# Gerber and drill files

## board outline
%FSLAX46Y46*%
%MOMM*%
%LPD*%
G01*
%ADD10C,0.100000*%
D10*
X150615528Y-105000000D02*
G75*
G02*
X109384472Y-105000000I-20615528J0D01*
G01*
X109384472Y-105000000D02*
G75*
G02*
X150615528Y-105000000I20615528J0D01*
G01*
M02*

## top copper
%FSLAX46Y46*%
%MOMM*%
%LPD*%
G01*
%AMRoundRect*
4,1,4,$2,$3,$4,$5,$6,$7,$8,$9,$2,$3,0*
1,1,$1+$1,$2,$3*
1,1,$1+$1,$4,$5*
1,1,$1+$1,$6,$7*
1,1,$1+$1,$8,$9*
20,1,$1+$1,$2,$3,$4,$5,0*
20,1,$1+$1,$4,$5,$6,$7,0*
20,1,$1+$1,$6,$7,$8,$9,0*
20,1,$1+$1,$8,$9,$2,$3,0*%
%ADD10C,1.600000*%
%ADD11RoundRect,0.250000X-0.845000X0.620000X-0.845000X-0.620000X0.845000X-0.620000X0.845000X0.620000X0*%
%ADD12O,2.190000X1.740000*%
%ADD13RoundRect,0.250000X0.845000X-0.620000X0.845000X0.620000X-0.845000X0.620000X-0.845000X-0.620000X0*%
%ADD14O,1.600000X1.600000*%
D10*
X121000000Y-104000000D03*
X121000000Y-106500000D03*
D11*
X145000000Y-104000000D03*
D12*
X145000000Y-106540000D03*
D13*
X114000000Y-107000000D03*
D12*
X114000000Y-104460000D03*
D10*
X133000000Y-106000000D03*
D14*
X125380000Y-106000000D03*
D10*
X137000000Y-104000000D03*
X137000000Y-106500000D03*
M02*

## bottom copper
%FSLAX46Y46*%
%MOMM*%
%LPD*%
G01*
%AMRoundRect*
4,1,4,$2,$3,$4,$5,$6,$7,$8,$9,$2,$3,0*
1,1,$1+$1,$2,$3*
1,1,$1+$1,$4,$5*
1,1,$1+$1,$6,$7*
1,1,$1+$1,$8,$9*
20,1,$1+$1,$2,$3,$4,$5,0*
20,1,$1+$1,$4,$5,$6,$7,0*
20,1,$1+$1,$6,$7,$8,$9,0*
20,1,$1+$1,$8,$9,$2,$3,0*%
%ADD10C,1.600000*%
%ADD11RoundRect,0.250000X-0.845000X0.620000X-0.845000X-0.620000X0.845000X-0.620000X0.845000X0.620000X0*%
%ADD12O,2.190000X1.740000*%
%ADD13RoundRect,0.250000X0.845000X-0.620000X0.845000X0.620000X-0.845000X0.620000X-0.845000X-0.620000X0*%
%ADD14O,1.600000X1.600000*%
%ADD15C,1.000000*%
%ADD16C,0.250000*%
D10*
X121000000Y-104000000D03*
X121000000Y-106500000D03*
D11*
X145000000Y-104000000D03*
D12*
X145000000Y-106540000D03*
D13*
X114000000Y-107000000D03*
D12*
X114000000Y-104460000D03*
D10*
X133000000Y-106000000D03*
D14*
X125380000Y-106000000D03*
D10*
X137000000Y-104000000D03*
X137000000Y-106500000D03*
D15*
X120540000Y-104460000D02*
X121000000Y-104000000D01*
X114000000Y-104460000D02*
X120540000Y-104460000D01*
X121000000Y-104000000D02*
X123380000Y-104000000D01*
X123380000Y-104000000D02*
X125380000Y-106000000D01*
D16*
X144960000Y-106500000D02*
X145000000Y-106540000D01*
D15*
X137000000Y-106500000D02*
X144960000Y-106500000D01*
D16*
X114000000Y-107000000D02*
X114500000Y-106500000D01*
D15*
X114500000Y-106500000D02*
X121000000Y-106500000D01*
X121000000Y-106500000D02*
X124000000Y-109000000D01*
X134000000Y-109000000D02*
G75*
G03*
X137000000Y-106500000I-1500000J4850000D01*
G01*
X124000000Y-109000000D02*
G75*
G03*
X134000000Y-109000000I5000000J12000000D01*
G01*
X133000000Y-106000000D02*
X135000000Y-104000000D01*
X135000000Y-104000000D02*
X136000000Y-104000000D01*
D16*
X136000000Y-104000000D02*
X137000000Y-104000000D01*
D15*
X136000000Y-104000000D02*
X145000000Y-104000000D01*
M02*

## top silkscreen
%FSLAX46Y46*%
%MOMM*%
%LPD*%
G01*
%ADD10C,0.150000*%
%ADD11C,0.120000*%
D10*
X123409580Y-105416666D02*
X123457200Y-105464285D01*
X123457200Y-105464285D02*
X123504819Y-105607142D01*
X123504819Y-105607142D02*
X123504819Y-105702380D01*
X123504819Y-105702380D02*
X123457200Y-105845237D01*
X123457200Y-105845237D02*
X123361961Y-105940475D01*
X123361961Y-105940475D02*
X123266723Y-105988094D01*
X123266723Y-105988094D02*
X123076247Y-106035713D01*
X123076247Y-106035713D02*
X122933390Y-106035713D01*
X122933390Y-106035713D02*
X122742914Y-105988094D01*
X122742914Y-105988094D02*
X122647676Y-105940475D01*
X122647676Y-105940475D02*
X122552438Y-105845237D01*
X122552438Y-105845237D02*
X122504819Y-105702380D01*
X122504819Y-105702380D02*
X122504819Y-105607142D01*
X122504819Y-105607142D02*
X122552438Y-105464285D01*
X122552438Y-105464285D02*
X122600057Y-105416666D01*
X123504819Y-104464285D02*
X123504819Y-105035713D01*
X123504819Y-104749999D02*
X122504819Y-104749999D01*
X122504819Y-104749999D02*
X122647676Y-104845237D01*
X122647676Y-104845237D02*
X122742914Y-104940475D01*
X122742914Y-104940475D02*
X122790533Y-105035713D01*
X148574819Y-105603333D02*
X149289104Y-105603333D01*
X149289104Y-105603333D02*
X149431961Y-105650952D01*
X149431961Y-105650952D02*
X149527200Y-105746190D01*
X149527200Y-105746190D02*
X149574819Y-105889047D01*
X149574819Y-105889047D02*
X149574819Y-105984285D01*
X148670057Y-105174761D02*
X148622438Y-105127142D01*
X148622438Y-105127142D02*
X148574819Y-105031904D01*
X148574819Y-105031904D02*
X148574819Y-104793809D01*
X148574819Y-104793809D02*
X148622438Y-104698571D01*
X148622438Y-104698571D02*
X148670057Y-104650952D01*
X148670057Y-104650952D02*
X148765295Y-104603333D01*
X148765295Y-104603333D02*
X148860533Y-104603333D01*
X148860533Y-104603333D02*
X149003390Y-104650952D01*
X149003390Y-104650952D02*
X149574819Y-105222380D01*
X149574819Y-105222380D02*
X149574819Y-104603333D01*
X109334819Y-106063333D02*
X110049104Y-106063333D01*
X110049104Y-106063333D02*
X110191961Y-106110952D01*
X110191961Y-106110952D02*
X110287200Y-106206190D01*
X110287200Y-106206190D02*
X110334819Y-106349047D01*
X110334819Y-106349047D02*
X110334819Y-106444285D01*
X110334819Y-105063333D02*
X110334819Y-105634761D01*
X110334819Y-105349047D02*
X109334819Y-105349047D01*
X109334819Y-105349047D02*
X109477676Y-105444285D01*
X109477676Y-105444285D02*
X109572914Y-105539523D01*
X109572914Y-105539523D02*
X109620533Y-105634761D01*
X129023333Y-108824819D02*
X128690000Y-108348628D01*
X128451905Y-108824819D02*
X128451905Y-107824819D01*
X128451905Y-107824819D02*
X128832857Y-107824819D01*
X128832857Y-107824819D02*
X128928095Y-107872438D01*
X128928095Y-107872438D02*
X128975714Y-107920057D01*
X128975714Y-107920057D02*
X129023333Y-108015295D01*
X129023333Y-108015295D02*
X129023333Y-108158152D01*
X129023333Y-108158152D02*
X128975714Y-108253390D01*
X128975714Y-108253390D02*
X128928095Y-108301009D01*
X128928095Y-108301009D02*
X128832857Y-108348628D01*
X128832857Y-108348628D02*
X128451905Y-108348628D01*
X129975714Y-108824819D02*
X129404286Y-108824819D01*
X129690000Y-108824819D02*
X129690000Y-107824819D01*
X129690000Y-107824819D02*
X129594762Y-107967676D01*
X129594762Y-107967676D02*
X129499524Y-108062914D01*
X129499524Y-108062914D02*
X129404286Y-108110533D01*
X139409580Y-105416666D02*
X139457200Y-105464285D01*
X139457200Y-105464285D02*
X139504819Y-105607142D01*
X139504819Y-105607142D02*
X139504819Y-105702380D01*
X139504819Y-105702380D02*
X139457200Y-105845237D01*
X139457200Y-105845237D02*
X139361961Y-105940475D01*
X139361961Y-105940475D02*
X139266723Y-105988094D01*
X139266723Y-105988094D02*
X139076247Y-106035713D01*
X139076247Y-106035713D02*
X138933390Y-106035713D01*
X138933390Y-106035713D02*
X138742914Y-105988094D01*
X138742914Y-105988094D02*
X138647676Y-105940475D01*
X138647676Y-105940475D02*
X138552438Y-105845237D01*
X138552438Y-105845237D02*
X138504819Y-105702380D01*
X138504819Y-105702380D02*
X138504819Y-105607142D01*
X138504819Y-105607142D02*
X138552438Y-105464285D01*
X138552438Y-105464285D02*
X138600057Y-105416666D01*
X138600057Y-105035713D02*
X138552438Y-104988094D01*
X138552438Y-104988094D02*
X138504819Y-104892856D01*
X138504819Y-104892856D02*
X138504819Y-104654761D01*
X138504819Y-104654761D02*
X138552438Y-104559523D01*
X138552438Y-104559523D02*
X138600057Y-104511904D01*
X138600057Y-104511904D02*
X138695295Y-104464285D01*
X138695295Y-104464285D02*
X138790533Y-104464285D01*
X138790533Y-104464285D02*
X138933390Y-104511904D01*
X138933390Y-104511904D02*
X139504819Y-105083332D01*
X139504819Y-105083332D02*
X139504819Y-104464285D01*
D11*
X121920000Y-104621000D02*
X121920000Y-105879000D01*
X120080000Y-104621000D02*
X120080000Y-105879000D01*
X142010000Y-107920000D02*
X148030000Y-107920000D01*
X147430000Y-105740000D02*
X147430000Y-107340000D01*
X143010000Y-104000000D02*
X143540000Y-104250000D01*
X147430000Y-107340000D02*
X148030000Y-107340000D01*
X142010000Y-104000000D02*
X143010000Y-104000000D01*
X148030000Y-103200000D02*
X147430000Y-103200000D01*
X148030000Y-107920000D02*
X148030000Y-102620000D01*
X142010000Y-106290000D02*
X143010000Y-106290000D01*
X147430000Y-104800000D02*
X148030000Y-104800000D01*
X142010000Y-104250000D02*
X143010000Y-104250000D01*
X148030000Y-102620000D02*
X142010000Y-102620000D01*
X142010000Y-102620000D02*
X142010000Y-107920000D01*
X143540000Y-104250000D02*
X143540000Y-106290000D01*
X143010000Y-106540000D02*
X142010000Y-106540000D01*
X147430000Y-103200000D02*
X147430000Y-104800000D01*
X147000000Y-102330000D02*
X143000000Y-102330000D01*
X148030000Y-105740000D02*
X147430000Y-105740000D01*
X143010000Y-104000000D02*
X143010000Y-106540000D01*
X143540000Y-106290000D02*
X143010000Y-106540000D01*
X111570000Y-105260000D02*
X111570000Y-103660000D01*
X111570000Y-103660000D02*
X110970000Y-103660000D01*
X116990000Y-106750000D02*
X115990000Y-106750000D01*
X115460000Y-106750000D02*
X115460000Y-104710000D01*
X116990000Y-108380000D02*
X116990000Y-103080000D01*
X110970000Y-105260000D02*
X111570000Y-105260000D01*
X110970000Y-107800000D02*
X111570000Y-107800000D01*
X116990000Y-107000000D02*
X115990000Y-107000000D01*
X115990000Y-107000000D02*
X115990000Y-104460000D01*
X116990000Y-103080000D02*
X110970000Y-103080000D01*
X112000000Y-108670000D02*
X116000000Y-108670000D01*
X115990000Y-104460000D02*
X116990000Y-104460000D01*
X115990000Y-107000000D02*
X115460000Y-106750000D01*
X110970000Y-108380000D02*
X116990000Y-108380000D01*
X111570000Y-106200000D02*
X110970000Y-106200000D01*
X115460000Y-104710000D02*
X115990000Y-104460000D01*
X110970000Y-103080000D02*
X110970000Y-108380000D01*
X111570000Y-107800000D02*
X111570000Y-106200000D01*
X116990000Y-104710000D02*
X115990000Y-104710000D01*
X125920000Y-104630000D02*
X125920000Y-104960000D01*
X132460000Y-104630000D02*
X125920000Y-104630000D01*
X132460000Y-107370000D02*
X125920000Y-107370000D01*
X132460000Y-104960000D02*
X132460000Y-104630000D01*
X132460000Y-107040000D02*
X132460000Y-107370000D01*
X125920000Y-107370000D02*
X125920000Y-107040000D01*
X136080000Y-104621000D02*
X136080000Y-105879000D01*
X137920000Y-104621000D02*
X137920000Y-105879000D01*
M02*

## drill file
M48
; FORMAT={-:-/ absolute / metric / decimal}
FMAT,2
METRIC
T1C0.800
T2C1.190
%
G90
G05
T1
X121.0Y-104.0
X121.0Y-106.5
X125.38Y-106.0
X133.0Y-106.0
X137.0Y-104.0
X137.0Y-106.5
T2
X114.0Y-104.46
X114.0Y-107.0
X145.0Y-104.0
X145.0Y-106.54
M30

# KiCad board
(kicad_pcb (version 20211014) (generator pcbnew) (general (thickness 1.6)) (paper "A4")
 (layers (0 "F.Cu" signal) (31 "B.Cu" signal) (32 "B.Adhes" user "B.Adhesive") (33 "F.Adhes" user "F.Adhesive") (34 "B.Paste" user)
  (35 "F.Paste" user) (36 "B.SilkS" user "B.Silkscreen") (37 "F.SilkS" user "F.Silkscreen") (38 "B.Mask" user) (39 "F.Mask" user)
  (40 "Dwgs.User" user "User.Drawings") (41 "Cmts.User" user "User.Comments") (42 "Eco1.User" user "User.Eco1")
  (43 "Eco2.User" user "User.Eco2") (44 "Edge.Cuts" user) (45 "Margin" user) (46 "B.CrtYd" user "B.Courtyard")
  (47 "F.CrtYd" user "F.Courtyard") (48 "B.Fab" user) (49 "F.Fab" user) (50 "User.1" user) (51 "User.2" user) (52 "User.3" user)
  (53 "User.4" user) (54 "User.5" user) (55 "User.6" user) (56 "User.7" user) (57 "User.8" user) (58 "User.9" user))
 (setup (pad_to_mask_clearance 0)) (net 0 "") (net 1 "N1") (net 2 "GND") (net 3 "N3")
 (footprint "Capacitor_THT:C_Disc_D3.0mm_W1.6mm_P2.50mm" (layer "F.Cu") (at 121 104 -90)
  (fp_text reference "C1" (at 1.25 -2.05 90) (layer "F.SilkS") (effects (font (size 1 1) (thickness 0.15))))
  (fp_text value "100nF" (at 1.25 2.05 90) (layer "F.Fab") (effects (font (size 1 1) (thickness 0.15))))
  (fp_line (start 0.621 -0.92) (end 1.879 -0.92) (layer "F.SilkS") (width 0.12))
  (fp_line (start 0.621 0.92) (end 1.879 0.92) (layer "F.SilkS") (width 0.12))
  (pad "1" thru_hole circle (at 0 0 270) (size 1.6 1.6) (drill 0.8) (layers *.Cu *.Mask) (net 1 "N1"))
  (pad "2" thru_hole circle (at 2.5 0 270) (size 1.6 1.6) (drill 0.8) (layers *.Cu *.Mask) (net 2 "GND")))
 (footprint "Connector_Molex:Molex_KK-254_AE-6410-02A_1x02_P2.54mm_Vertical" (layer "F.Cu") (at 145 104 -90)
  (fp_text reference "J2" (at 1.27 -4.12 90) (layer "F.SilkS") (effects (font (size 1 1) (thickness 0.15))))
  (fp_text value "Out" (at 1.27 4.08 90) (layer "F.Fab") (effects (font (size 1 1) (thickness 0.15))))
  (fp_line (start 3.92 2.99) (end 3.92 -3.03) (layer "F.SilkS") (width 0.12))
  (fp_line (start 1.74 -2.43) (end 3.34 -2.43) (layer "F.SilkS") (width 0.12))
  (fp_line (start 0 1.99) (end 0.25 1.46) (layer "F.SilkS") (width 0.12))
  (fp_line (start 3.34 -2.43) (end 3.34 -3.03) (layer "F.SilkS") (width 0.12))
  (fp_line (start 0 2.99) (end 0 1.99) (layer "F.SilkS") (width 0.12))
  (fp_line (start -0.8 -3.03) (end -0.8 -2.43) (layer "F.SilkS") (width 0.12))
  (fp_line (start 3.92 -3.03) (end -1.38 -3.03) (layer "F.SilkS") (width 0.12))
  (fp_line (start 2.29 2.99) (end 2.29 1.99) (layer "F.SilkS") (width 0.12))
  (fp_line (start 0.8 -2.43) (end 0.8 -3.03) (layer "F.SilkS") (width 0.12))
  (fp_line (start 0.25 2.99) (end 0.25 1.99) (layer "F.SilkS") (width 0.12))
  (fp_line (start -1.38 -3.03) (end -1.38 2.99) (layer "F.SilkS") (width 0.12))
  (fp_line (start -1.38 2.99) (end 3.92 2.99) (layer "F.SilkS") (width 0.12))
  (fp_line (start 0.25 1.46) (end 2.29 1.46) (layer "F.SilkS") (width 0.12))
  (fp_line (start 2.54 1.99) (end 2.54 2.99) (layer "F.SilkS") (width 0.12))
  (fp_line (start -0.8 -2.43) (end 0.8 -2.43) (layer "F.SilkS") (width 0.12))
  (fp_line (start -1.67 -2) (end -1.67 2) (layer "F.SilkS") (width 0.12))
  (fp_line (start 1.74 -3.03) (end 1.74 -2.43) (layer "F.SilkS") (width 0.12))
  (fp_line (start 0 1.99) (end 2.54 1.99) (layer "F.SilkS") (width 0.12))
  (fp_line (start 2.29 1.46) (end 2.54 1.99) (layer "F.SilkS") (width 0.12))
  (pad "1" thru_hole roundrect (at 0 0 270) (size 1.74 2.19) (drill 1.19) (layers *.Cu *.Mask) (roundrect_rratio 0.143678) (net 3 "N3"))
  (pad "2" thru_hole oval (at 2.54 0 270) (size 1.74 2.19) (drill 1.19) (layers *.Cu *.Mask) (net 2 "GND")))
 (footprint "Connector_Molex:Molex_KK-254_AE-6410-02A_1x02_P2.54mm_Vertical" (layer "F.Cu") (at 114 107 90)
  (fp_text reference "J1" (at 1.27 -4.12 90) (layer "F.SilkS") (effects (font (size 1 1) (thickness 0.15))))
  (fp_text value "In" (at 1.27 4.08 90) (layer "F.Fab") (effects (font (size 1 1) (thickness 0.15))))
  (fp_line (start 1.74 -2.43) (end 3.34 -2.43) (layer "F.SilkS") (width 0.12))
  (fp_line (start 3.34 -2.43) (end 3.34 -3.03) (layer "F.SilkS") (width 0.12))
  (fp_line (start 0.25 2.99) (end 0.25 1.99) (layer "F.SilkS") (width 0.12))
  (fp_line (start 0.25 1.46) (end 2.29 1.46) (layer "F.SilkS") (width 0.12))
  (fp_line (start -1.38 2.99) (end 3.92 2.99) (layer "F.SilkS") (width 0.12))
  (fp_line (start 1.74 -3.03) (end 1.74 -2.43) (layer "F.SilkS") (width 0.12))
  (fp_line (start -0.8 -3.03) (end -0.8 -2.43) (layer "F.SilkS") (width 0.12))
  (fp_line (start 0 2.99) (end 0 1.99) (layer "F.SilkS") (width 0.12))
  (fp_line (start 0 1.99) (end 2.54 1.99) (layer "F.SilkS") (width 0.12))
  (fp_line (start 3.92 2.99) (end 3.92 -3.03) (layer "F.SilkS") (width 0.12))
  (fp_line (start -1.67 -2) (end -1.67 2) (layer "F.SilkS") (width 0.12))
  (fp_line (start 2.54 1.99) (end 2.54 2.99) (layer "F.SilkS") (width 0.12))
  (fp_line (start 0 1.99) (end 0.25 1.46) (layer "F.SilkS") (width 0.12))
  (fp_line (start -1.38 -3.03) (end -1.38 2.99) (layer "F.SilkS") (width 0.12))
  (fp_line (start 0.8 -2.43) (end 0.8 -3.03) (layer "F.SilkS") (width 0.12))
  (fp_line (start 2.29 1.46) (end 2.54 1.99) (layer "F.SilkS") (width 0.12))
  (fp_line (start 3.92 -3.03) (end -1.38 -3.03) (layer "F.SilkS") (width 0.12))
  (fp_line (start -0.8 -2.43) (end 0.8 -2.43) (layer "F.SilkS") (width 0.12))
  (fp_line (start 2.29 2.99) (end 2.29 1.99) (layer "F.SilkS") (width 0.12))
  (pad "1" thru_hole roundrect (at 0 0 90) (size 1.74 2.19) (drill 1.19) (layers *.Cu *.Mask) (roundrect_rratio 0.143678) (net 2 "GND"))
  (pad "2" thru_hole oval (at 2.54 0 90) (size 1.74 2.19) (drill 1.19) (layers *.Cu *.Mask) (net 1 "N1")))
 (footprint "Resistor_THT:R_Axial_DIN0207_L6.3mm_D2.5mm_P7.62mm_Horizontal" (layer "F.Cu") (at 133 106 180)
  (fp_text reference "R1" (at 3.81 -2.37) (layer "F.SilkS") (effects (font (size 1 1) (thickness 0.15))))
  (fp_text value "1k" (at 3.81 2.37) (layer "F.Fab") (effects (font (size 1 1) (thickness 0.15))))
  (fp_line (start 7.08 1.37) (end 7.08 1.04) (layer "F.SilkS") (width 0.12))
  (fp_line (start 0.54 1.37) (end 7.08 1.37) (layer "F.SilkS") (width 0.12))
  (fp_line (start 0.54 -1.37) (end 7.08 -1.37) (layer "F.SilkS") (width 0.12))
  (fp_line (start 0.54 1.04) (end 0.54 1.37) (layer "F.SilkS") (width 0.12))
  (fp_line (start 0.54 -1.04) (end 0.54 -1.37) (layer "F.SilkS") (width 0.12))
  (fp_line (start 7.08 -1.37) (end 7.08 -1.04) (layer "F.SilkS") (width 0.12))
  (pad "1" thru_hole circle (at 0 0 180) (size 1.6 1.6) (drill 0.8) (layers *.Cu *.Mask) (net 3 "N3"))
  (pad "2" thru_hole oval (at 7.62 0 180) (size 1.6 1.6) (drill 0.8) (layers *.Cu *.Mask) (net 1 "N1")))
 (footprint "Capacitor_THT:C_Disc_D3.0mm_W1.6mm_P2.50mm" (layer "F.Cu") (at 137 104 -90)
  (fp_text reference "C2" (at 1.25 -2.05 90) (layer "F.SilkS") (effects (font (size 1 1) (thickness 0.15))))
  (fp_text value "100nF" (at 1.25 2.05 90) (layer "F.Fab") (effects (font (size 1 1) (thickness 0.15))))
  (fp_line (start 0.621 0.92) (end 1.879 0.92) (layer "F.SilkS") (width 0.12))
  (fp_line (start 0.621 -0.92) (end 1.879 -0.92) (layer "F.SilkS") (width 0.12))
  (pad "1" thru_hole circle (at 0 0 270) (size 1.6 1.6) (drill 0.8) (layers *.Cu *.Mask) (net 3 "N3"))
  (pad "2" thru_hole circle (at 2.5 0 270) (size 1.6 1.6) (drill 0.8) (layers *.Cu *.Mask) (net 2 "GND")))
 (gr_circle (center 130 105) (end 110 110) (layer "Edge.Cuts") (width 0.1) (fill none))
 (segment (start 120.54 104.46) (end 121 104) (width 1) (layer "B.Cu") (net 1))
 (segment (start 114 104.46) (end 120.54 104.46) (width 1) (layer "B.Cu") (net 1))
 (segment (start 121 104) (end 123.38 104) (width 1) (layer "B.Cu") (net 1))
 (segment (start 123.38 104) (end 125.38 106) (width 1) (layer "B.Cu") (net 1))
 (segment (start 144.96 106.5) (end 145 106.54) (width 0.25) (layer "B.Cu") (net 2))
 (segment (start 137 106.5) (end 144.96 106.5) (width 1) (layer "B.Cu") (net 2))
 (segment (start 114 107) (end 114.5 106.5) (width 0.25) (layer "B.Cu") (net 2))
 (segment (start 114.5 106.5) (end 121 106.5) (width 1) (layer "B.Cu") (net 2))
 (segment (start 121 106.5) (end 124 109) (width 1) (layer "B.Cu") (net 2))
 (arc (start 134 109) (mid 135.75 108.05) (end 137 106.5) (width 1) (layer "B.Cu") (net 2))
 (arc (start 124 109) (mid 129 110) (end 134 109) (width 1) (layer "B.Cu") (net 2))
 (segment (start 133 106) (end 135 104) (width 1) (layer "B.Cu") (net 3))
 (segment (start 135 104) (end 136 104) (width 1) (layer "B.Cu") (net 3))
 (segment (start 136 104) (end 137 104) (width 0.25) (layer "B.Cu") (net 3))
 (segment (start 136 104) (end 145 104) (width 1) (layer "B.Cu") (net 3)))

